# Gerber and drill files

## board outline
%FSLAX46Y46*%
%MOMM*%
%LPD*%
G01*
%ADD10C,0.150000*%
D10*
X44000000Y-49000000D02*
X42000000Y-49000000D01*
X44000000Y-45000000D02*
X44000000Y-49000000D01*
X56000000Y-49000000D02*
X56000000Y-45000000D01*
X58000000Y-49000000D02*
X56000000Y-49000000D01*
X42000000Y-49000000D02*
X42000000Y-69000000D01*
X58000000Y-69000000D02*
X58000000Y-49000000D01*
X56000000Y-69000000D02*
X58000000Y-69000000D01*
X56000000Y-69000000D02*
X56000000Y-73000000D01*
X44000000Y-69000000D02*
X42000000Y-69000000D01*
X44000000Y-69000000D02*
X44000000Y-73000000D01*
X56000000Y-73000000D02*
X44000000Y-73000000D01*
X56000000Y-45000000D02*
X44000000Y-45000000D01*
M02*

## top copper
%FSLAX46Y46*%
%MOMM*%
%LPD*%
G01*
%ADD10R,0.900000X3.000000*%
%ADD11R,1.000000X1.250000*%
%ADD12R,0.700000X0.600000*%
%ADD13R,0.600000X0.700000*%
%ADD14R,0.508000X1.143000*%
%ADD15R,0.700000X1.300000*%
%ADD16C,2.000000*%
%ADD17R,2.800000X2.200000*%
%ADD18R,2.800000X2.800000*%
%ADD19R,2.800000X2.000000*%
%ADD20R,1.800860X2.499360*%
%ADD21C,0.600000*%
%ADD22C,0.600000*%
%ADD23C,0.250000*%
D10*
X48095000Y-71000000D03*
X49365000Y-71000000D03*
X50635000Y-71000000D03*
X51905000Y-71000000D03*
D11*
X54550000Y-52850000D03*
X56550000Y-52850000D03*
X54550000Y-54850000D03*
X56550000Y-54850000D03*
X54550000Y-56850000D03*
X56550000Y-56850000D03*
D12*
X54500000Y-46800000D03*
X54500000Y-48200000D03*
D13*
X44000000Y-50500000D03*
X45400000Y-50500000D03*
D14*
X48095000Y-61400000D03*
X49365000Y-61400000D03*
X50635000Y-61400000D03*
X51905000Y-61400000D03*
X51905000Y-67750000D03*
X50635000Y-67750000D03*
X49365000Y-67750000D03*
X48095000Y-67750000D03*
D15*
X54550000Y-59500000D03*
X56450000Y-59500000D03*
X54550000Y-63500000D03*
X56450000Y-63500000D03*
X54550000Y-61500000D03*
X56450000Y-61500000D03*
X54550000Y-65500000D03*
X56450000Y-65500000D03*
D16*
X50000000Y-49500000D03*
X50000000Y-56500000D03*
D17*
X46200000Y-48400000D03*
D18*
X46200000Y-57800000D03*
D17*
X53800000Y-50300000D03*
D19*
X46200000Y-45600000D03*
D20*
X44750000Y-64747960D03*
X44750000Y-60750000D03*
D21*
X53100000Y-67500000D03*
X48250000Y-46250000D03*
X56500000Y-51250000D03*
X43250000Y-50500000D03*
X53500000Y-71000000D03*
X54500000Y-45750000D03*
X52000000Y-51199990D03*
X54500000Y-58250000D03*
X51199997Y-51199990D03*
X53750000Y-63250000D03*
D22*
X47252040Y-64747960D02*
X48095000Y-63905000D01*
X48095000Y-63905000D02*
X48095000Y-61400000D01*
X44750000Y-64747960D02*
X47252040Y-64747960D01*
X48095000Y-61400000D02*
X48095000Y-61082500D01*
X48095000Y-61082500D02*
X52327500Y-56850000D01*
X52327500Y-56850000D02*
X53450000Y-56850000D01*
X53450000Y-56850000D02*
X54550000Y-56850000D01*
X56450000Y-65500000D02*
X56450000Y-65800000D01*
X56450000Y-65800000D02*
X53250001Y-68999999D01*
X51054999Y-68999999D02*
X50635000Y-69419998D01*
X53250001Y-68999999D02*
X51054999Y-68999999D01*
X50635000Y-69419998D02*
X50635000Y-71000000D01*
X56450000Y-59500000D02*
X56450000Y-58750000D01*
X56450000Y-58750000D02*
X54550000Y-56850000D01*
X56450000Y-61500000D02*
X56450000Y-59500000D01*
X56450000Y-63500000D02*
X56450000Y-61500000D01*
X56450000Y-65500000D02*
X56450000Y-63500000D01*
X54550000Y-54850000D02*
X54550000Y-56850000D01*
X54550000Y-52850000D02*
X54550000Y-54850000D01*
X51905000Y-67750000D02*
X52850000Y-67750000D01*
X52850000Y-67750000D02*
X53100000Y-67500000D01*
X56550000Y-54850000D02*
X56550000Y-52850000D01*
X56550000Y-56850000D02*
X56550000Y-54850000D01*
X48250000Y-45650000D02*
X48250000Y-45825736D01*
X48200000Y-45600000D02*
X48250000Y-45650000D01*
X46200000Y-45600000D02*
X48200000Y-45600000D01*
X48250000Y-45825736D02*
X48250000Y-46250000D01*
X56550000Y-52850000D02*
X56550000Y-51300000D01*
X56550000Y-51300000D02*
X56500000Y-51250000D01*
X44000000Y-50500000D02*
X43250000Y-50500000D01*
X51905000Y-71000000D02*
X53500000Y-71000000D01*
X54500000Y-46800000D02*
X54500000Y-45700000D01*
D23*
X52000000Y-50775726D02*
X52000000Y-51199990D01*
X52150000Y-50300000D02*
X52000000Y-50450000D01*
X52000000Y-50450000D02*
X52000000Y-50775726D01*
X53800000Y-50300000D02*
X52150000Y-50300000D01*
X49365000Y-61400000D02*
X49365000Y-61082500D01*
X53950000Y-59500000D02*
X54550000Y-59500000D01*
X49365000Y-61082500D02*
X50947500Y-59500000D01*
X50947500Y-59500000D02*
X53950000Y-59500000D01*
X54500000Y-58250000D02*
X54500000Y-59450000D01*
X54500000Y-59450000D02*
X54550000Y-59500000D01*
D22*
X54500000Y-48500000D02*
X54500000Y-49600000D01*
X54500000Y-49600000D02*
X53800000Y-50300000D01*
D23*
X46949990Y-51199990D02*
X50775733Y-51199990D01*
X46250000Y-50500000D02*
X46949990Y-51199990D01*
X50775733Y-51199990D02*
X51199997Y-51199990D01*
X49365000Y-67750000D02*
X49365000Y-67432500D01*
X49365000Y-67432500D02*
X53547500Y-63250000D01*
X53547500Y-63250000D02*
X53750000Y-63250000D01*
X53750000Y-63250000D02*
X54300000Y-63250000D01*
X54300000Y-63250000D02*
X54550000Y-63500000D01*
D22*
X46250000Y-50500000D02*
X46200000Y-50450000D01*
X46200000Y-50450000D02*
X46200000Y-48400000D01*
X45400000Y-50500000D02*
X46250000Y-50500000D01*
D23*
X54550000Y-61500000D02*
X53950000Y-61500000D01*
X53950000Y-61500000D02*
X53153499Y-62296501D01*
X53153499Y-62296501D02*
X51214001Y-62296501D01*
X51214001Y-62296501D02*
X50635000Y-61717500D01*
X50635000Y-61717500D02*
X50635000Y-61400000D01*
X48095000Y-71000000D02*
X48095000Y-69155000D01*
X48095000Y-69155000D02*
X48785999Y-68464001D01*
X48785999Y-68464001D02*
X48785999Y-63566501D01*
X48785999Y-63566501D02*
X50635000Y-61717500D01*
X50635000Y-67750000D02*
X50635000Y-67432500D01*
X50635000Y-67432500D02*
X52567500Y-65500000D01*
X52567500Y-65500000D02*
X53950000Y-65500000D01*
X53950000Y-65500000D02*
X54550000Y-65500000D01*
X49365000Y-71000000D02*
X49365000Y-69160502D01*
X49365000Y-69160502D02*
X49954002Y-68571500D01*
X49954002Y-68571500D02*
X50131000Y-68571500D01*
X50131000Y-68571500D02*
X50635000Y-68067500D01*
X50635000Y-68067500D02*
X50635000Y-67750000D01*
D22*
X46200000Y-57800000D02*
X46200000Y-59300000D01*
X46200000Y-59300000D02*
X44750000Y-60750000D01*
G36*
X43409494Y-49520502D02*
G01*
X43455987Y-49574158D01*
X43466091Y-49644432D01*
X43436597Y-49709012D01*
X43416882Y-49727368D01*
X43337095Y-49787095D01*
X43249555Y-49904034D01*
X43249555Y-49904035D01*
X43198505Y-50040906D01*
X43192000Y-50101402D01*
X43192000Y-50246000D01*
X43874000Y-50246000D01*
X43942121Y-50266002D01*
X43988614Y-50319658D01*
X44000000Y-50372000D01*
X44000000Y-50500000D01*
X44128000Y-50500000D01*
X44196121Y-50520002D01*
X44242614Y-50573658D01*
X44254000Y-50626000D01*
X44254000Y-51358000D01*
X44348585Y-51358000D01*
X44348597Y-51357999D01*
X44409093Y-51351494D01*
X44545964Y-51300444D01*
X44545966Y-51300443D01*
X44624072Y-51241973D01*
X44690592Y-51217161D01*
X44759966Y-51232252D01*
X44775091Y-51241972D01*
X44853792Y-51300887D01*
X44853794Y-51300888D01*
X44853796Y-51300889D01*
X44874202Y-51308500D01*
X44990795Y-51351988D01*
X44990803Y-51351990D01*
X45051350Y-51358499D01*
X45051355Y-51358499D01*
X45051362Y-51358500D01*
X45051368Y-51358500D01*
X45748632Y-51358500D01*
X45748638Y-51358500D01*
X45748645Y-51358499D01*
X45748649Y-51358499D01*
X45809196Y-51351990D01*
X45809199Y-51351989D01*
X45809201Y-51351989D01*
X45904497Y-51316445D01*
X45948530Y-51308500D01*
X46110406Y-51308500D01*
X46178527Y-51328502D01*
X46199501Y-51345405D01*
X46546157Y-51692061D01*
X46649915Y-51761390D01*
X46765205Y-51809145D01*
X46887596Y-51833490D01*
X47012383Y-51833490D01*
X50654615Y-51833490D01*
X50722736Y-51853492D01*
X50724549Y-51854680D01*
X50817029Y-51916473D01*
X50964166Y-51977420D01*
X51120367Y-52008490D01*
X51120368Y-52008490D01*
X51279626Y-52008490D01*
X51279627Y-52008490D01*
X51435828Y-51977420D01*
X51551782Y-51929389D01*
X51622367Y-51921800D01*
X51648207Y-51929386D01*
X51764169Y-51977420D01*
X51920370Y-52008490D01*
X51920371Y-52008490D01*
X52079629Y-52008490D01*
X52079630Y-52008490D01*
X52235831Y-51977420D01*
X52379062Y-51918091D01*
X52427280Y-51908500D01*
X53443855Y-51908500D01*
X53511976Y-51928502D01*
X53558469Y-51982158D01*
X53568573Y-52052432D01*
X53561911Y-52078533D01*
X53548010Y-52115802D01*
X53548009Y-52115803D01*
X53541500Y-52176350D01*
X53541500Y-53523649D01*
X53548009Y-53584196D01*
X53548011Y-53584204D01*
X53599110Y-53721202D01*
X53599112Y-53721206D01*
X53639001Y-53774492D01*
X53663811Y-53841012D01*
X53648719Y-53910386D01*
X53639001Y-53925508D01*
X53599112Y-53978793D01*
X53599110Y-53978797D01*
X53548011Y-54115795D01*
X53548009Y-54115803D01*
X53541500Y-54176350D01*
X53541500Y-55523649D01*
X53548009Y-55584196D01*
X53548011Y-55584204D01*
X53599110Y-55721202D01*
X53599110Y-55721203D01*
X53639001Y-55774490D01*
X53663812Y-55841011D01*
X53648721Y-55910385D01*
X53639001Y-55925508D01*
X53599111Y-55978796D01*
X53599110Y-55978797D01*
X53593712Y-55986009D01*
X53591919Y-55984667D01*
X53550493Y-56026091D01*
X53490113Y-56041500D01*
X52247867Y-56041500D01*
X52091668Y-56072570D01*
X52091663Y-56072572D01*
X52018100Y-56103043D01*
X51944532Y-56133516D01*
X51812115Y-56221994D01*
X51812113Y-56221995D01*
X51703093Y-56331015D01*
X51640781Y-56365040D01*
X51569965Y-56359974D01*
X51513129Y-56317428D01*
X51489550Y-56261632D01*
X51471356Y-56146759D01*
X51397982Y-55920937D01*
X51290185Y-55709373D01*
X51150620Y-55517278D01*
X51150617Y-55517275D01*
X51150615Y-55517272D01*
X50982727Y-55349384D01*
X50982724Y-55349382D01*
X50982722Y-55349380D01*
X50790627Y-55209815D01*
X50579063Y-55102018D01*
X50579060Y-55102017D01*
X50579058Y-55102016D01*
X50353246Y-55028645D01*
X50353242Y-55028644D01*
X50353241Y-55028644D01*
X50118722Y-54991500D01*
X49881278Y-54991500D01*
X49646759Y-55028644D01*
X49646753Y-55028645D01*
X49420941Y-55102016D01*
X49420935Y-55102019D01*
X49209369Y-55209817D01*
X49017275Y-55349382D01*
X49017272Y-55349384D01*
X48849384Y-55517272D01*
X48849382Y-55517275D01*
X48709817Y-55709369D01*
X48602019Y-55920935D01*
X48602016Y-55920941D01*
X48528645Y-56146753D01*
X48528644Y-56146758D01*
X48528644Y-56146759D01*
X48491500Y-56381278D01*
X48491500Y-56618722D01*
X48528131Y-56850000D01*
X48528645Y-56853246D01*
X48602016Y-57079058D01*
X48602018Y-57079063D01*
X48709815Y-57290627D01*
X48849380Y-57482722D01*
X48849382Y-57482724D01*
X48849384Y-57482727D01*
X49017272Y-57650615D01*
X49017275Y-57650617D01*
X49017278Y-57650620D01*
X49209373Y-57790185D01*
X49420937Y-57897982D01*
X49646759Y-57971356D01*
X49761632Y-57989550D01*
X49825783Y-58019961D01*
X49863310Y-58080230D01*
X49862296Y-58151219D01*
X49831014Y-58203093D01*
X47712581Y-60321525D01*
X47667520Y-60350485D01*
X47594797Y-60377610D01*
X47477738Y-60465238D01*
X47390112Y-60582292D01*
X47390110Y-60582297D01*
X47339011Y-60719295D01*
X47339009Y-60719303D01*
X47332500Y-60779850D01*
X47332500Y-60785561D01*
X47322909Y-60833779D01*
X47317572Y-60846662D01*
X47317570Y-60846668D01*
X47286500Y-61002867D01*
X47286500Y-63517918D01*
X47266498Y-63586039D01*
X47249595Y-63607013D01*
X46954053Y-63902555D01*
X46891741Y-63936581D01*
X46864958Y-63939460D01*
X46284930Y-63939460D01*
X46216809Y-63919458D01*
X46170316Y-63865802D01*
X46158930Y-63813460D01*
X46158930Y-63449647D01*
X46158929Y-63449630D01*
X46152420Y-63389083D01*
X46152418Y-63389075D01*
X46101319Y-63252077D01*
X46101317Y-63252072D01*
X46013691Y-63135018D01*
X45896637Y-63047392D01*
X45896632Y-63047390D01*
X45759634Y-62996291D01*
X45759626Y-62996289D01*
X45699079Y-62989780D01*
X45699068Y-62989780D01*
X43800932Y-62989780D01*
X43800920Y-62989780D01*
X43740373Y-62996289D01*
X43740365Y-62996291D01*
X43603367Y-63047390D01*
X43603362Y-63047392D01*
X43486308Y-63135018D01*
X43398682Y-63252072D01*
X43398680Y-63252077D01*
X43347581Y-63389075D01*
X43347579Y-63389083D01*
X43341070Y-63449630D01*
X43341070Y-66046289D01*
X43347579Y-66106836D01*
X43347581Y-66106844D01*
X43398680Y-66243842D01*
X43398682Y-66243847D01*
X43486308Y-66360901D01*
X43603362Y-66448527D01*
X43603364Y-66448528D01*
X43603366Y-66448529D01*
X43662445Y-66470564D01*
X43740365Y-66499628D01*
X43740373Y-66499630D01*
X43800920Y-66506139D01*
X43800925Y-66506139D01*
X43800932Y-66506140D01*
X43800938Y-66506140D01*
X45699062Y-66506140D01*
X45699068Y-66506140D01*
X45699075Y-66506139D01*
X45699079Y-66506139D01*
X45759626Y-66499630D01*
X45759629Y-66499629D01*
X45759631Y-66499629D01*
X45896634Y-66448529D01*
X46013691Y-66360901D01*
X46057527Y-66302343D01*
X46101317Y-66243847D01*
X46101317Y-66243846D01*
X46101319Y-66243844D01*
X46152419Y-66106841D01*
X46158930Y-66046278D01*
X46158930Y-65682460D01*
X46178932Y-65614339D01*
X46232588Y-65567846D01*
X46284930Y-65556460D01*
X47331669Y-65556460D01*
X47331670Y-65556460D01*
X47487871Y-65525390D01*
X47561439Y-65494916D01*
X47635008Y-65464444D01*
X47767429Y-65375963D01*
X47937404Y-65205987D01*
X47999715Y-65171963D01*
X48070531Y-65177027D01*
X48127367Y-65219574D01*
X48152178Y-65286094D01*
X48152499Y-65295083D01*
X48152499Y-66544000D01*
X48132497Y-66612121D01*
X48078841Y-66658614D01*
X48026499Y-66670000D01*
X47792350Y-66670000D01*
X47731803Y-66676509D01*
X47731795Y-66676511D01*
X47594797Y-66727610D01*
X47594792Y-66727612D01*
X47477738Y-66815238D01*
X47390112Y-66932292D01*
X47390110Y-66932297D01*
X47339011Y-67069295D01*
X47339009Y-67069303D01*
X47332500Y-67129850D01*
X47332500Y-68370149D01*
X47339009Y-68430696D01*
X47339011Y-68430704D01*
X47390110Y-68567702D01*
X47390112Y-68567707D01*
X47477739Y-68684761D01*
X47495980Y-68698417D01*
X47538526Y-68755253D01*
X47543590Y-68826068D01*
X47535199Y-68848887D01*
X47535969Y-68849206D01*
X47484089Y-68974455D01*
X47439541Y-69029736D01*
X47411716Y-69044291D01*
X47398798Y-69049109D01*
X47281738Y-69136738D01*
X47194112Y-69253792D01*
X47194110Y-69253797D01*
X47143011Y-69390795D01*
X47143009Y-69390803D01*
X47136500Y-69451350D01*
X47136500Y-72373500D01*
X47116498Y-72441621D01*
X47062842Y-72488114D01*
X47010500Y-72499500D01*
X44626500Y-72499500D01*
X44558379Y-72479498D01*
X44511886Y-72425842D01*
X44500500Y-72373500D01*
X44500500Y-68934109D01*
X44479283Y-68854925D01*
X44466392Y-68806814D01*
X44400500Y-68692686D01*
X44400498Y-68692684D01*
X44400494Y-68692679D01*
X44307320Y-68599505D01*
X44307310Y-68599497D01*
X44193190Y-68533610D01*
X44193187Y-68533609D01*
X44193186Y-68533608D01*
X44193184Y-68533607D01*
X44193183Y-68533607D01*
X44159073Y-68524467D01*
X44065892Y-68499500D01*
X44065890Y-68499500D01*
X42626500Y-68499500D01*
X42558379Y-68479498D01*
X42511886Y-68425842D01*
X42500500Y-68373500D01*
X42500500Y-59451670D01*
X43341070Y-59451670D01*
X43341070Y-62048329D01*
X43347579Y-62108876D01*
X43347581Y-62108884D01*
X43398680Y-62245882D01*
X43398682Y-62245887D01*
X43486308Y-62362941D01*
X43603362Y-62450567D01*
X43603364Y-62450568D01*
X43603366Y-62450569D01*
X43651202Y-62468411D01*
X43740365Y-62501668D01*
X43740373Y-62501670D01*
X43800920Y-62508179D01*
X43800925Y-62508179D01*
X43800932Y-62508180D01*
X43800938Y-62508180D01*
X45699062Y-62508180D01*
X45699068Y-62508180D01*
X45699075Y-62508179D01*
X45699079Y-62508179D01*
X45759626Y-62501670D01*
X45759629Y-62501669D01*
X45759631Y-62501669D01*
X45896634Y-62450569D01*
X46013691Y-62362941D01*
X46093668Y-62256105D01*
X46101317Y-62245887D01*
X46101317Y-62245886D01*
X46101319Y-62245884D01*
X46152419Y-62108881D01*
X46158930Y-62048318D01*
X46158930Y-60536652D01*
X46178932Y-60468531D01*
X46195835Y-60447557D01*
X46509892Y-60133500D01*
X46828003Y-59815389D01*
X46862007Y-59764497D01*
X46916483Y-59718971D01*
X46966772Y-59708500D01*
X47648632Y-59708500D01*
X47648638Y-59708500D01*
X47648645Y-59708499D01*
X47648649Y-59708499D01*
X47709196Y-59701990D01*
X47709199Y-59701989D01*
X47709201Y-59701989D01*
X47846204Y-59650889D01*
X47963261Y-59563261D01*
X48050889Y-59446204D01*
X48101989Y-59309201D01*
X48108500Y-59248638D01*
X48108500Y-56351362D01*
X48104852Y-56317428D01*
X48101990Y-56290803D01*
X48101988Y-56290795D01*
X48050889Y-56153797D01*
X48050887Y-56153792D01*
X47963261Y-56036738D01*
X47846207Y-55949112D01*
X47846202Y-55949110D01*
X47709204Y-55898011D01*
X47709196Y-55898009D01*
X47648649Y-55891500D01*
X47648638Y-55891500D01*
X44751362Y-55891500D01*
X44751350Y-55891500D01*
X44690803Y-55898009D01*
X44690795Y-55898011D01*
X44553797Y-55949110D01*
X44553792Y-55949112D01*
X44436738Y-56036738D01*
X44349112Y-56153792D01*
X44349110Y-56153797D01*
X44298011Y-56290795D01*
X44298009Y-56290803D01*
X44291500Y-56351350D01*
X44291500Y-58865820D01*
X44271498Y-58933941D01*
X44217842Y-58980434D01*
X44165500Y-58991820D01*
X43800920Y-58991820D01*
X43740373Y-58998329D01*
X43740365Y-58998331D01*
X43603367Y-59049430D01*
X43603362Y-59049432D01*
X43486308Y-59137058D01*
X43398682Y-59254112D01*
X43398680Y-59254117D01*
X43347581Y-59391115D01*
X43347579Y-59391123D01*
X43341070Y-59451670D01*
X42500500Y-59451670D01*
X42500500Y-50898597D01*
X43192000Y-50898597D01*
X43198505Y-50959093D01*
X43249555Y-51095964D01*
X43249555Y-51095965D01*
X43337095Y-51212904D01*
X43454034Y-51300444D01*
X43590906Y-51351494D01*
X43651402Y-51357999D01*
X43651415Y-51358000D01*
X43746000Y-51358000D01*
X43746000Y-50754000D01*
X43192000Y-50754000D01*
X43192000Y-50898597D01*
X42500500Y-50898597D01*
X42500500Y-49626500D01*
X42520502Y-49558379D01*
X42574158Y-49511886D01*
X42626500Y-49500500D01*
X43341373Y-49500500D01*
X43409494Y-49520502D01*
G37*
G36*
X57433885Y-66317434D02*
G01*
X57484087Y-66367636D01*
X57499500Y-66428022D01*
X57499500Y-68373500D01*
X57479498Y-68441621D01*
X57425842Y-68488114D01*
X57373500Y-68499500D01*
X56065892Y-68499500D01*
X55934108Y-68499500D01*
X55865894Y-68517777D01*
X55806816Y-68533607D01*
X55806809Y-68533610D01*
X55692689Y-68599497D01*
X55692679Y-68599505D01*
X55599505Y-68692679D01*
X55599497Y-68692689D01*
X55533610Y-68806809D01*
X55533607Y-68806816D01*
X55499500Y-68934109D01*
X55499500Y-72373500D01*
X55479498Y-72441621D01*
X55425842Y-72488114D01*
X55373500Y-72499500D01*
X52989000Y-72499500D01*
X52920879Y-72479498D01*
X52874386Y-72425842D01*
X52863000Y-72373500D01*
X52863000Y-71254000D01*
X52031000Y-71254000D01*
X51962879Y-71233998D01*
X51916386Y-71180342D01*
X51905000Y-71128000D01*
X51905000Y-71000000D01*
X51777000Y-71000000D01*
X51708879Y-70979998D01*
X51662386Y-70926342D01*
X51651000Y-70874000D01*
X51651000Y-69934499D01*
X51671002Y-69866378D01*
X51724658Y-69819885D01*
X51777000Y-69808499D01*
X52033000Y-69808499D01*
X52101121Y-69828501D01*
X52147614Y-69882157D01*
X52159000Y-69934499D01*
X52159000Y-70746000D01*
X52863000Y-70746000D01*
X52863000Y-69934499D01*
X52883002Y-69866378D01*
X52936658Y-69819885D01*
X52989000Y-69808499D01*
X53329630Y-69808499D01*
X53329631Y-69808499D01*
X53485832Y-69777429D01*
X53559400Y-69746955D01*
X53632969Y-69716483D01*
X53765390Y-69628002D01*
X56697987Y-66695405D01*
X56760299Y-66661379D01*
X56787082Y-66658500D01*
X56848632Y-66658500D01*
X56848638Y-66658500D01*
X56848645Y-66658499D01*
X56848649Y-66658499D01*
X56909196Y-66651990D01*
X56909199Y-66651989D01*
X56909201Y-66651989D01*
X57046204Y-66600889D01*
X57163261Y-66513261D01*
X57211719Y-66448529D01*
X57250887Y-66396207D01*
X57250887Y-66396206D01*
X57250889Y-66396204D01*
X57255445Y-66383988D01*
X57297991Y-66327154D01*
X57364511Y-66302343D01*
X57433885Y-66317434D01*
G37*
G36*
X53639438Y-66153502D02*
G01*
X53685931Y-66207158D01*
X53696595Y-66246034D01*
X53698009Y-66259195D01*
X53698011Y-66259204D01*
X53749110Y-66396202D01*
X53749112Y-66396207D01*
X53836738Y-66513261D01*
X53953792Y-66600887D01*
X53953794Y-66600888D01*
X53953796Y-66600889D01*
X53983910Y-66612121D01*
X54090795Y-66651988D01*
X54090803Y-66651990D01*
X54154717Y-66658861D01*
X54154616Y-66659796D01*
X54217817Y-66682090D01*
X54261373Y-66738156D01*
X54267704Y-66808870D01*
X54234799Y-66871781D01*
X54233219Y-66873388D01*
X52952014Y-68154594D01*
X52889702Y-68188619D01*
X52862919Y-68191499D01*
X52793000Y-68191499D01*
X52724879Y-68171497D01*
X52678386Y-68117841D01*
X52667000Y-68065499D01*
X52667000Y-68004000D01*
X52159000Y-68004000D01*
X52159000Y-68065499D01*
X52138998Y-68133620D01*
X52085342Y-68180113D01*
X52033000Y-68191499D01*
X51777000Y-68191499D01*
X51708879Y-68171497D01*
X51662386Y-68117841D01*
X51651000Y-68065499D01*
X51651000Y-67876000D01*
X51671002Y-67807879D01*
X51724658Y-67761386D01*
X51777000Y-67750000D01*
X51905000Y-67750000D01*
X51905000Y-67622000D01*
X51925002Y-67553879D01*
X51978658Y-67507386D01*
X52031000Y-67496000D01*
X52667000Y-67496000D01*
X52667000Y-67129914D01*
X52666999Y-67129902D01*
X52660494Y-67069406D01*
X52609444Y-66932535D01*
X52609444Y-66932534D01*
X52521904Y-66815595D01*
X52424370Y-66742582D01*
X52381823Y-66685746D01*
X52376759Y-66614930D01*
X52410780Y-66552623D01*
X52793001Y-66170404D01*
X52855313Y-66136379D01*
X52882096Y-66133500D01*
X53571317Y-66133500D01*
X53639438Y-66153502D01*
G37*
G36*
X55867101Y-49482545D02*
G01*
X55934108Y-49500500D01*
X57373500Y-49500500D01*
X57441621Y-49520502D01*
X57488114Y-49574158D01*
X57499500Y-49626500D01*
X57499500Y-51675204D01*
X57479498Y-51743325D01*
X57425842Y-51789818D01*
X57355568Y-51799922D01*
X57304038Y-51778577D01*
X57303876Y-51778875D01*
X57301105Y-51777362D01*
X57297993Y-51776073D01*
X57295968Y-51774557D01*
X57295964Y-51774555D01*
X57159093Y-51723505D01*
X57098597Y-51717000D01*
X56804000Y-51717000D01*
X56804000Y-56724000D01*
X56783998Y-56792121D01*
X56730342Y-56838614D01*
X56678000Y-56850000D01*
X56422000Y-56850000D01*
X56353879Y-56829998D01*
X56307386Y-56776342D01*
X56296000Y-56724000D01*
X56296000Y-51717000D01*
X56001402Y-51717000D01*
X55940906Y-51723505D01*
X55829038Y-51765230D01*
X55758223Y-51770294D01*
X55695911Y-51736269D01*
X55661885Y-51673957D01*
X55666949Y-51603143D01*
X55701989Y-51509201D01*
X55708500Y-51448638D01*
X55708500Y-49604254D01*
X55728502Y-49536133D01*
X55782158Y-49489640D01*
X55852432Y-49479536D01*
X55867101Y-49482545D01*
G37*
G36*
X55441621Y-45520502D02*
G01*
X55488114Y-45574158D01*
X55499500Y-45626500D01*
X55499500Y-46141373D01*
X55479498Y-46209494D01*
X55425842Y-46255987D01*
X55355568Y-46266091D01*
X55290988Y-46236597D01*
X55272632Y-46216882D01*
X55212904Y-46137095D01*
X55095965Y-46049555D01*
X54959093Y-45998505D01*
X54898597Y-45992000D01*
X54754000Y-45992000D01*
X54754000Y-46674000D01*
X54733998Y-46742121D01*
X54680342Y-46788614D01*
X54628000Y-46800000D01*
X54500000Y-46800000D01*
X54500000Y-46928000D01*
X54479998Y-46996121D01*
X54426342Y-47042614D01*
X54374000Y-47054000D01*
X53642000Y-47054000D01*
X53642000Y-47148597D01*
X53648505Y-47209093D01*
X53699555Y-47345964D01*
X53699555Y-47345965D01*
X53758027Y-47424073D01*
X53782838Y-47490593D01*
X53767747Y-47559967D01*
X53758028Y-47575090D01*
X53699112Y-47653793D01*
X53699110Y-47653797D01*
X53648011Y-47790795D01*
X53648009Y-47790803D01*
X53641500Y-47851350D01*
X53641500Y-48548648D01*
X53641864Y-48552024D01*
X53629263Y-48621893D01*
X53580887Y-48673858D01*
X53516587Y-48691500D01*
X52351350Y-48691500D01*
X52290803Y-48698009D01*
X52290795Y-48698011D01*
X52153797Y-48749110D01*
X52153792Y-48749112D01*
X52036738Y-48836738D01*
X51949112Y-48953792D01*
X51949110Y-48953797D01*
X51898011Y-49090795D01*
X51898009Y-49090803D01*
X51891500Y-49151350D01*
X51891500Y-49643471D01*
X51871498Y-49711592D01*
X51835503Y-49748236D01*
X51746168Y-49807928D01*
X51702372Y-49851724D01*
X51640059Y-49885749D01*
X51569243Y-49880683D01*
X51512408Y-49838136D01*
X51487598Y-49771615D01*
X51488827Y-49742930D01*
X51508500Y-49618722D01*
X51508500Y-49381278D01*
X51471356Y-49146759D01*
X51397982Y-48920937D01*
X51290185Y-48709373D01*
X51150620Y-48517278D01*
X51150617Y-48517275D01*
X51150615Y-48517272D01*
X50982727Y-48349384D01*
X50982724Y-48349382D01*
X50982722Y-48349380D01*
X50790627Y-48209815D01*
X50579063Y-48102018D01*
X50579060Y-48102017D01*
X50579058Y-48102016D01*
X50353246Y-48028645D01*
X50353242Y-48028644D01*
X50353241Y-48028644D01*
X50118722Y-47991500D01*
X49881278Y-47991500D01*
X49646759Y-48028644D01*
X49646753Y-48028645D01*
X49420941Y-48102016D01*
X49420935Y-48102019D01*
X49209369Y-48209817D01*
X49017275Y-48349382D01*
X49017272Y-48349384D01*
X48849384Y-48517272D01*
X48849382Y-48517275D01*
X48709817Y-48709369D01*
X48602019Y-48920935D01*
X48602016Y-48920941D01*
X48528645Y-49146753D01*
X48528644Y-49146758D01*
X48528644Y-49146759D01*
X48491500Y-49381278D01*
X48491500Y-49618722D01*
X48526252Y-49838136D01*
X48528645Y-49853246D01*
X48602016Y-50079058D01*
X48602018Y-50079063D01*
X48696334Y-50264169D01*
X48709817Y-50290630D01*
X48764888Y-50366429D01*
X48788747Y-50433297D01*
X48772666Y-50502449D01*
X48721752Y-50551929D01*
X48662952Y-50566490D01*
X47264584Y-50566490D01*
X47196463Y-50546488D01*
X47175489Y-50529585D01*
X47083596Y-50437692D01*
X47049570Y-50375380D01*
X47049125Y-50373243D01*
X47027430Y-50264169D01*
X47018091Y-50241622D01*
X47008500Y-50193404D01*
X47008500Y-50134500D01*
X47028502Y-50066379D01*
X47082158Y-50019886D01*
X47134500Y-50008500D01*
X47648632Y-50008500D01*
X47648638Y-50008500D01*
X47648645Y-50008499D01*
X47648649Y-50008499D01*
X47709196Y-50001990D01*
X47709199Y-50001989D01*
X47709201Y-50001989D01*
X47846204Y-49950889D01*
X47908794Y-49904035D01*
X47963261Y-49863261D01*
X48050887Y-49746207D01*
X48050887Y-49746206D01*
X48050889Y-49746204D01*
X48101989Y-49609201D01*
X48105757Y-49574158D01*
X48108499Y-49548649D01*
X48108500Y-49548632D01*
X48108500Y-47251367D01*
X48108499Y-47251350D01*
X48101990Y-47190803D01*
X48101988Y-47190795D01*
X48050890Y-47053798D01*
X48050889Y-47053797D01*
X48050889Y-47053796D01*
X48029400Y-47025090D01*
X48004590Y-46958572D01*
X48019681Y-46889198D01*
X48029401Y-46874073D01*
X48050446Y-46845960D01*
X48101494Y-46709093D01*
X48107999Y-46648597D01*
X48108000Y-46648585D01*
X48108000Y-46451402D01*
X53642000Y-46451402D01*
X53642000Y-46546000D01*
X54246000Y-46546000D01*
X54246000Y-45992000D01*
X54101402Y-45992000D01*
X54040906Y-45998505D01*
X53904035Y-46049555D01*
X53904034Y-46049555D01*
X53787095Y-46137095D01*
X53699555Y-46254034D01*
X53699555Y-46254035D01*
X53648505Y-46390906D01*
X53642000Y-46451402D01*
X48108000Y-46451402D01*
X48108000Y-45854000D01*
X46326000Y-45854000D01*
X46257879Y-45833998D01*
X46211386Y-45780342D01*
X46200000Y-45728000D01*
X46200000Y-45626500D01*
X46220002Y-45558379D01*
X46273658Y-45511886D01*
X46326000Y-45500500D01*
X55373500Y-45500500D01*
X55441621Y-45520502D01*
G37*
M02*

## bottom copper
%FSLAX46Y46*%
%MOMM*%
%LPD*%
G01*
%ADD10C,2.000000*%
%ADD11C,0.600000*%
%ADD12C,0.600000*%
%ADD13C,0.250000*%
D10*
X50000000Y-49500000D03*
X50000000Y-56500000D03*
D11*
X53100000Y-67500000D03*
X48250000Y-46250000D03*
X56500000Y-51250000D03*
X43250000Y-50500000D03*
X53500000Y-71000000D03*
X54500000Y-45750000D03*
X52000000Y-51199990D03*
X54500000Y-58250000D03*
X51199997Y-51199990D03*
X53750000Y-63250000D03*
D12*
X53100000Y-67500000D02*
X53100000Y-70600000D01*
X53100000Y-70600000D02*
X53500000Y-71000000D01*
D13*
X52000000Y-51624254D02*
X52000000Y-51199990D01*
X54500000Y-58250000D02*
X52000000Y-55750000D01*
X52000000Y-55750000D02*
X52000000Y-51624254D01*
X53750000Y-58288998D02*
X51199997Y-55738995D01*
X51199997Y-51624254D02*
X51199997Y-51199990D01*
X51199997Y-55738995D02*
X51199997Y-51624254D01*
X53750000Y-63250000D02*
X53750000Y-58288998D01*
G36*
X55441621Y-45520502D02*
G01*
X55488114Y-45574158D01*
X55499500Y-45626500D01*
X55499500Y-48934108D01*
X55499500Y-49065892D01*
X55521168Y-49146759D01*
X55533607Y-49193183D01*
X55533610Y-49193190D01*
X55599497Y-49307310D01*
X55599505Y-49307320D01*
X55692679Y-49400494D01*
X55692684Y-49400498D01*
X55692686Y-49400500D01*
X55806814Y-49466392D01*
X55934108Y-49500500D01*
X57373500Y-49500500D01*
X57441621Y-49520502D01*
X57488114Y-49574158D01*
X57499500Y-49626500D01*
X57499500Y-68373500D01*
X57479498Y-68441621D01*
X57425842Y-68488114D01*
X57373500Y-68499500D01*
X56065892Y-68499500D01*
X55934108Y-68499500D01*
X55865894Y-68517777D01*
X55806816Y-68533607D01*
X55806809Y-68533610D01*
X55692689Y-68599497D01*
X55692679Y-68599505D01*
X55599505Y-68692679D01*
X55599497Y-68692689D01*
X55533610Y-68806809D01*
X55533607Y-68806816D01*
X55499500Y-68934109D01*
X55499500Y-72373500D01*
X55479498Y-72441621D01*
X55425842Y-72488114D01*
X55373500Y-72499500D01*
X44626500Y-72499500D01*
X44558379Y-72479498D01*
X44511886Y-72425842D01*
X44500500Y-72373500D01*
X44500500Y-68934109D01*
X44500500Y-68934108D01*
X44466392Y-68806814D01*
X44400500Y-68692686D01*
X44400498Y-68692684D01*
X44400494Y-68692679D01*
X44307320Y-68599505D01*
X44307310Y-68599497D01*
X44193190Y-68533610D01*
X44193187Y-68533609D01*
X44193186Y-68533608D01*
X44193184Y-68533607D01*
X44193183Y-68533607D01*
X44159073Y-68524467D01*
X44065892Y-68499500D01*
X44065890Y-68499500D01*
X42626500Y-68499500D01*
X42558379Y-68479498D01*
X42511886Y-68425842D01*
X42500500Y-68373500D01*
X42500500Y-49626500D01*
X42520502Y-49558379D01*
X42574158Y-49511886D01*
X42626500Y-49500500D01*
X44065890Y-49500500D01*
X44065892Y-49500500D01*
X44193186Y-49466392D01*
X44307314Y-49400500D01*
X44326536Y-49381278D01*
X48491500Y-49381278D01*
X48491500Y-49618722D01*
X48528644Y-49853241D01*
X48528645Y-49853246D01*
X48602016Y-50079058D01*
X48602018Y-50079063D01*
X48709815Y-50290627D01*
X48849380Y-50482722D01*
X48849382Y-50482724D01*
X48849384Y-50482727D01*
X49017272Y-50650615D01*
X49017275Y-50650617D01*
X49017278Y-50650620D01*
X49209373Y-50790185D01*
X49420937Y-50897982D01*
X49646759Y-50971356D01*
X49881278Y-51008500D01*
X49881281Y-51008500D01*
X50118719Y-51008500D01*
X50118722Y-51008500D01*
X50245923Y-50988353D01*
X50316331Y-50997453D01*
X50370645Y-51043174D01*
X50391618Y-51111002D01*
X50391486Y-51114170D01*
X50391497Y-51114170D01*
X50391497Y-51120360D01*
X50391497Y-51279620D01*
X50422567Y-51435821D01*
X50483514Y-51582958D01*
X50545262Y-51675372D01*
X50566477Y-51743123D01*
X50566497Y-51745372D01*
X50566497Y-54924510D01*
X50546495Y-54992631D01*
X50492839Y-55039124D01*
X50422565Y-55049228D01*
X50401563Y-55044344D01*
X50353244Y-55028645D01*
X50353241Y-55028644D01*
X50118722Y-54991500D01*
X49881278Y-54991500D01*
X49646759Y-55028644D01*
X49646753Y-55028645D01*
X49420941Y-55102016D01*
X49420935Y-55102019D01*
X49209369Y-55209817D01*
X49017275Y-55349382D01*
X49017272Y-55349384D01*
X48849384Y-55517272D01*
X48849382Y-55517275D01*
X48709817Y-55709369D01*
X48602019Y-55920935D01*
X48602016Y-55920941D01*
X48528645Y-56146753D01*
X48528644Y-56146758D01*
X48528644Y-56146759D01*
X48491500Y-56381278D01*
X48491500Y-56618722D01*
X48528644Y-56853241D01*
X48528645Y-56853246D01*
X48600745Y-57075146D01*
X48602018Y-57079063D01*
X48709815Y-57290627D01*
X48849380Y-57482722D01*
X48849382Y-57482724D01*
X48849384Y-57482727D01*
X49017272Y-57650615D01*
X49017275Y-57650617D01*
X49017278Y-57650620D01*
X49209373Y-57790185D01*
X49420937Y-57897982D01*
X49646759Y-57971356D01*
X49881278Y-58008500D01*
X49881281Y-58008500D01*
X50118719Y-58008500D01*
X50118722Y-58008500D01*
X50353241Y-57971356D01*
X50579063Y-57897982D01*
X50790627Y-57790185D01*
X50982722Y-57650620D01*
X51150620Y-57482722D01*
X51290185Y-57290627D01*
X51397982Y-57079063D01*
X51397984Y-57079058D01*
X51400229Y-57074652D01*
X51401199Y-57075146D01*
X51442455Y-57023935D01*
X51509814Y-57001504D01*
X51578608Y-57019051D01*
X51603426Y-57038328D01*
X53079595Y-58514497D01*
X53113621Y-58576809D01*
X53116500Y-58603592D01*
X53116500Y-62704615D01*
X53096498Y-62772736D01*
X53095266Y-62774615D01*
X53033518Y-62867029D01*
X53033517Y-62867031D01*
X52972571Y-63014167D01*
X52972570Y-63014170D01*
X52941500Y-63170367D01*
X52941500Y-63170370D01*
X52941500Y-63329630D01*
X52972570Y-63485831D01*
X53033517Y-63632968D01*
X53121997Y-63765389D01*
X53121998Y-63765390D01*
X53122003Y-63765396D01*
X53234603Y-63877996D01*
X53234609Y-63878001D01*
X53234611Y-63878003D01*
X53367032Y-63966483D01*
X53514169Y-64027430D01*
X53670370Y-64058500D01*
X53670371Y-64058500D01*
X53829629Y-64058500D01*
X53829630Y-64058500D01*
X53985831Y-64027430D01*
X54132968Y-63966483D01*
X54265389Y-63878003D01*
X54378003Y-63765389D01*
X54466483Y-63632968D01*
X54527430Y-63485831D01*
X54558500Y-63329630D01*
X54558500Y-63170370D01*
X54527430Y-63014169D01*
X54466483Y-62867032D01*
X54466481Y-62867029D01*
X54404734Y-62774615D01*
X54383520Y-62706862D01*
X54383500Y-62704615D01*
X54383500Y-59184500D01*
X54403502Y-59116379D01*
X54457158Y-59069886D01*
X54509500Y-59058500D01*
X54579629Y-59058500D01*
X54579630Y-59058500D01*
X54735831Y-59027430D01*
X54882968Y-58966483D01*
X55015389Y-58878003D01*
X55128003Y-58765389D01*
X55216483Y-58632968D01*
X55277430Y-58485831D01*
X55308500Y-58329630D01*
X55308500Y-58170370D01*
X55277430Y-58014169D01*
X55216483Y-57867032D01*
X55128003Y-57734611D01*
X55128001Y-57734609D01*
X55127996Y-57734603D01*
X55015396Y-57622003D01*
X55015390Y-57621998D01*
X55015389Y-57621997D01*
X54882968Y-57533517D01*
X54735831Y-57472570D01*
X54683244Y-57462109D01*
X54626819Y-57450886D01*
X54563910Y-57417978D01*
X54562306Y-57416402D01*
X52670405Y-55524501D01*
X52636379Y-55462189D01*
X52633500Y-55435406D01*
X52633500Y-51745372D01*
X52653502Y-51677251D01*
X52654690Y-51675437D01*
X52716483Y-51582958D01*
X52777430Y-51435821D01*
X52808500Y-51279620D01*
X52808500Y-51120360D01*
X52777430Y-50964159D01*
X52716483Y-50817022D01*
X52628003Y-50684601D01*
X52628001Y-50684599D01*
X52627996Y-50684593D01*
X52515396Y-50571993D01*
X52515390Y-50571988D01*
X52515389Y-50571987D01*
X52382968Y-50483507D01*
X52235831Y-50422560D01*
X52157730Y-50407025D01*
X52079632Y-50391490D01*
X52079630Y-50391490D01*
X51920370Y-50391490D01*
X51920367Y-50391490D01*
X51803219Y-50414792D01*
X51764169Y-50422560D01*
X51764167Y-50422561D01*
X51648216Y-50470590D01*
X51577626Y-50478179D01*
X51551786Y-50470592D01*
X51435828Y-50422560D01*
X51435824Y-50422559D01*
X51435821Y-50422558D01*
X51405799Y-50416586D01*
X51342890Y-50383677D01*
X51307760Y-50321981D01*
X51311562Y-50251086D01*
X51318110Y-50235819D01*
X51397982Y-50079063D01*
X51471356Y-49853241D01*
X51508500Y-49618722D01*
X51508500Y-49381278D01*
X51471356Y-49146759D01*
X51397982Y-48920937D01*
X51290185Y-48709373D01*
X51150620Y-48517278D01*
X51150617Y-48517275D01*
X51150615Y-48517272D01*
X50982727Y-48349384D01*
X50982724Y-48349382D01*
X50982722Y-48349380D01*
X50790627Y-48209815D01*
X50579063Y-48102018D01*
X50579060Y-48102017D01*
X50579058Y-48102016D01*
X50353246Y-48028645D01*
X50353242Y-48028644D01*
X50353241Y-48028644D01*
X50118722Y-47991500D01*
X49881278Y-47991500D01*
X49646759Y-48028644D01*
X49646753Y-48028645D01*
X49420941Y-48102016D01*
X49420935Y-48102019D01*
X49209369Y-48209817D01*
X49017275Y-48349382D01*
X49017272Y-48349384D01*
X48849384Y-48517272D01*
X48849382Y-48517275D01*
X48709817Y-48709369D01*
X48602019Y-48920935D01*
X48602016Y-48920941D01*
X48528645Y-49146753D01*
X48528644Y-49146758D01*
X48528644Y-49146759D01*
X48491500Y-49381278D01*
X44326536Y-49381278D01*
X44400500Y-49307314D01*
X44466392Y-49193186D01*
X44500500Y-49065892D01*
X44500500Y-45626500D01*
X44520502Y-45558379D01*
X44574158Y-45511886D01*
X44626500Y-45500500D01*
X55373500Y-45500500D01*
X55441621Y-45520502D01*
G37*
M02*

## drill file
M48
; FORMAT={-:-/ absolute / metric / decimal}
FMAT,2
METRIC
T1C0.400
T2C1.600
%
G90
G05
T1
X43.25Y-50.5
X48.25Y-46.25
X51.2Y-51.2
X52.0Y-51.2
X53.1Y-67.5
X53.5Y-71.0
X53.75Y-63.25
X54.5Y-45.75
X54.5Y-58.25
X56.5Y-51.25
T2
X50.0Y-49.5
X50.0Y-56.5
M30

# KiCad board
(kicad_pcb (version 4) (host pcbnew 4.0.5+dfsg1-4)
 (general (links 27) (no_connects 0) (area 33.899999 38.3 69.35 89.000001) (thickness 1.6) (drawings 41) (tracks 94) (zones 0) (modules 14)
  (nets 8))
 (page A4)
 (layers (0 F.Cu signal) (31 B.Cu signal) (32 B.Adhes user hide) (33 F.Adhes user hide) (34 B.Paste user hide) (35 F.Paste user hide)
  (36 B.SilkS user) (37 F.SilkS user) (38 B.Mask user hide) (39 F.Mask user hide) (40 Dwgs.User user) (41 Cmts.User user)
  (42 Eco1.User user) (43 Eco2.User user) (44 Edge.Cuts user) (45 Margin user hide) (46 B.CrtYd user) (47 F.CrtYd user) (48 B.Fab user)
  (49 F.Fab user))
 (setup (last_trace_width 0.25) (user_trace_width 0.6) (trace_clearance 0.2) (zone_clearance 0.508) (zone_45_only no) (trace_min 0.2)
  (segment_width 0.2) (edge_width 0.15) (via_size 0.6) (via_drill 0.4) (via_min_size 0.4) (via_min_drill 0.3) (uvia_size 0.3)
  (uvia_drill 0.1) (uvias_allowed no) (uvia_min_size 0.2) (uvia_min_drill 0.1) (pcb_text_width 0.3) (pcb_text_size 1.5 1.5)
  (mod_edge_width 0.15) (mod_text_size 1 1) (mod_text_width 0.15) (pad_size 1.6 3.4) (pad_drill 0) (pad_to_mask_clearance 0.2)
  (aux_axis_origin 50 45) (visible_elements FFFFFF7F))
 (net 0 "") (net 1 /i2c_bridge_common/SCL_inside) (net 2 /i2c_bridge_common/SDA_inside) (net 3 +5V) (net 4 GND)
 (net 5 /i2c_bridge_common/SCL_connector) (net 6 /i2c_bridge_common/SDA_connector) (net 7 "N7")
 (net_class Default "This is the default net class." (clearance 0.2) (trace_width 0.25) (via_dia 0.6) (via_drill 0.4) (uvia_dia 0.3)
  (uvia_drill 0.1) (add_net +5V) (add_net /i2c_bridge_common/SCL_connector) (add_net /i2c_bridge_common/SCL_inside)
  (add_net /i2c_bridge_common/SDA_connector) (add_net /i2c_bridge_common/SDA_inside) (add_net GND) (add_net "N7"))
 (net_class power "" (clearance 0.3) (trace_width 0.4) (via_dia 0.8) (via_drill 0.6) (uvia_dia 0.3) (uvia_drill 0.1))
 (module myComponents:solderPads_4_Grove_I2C (layer F.Cu) (at 50 71)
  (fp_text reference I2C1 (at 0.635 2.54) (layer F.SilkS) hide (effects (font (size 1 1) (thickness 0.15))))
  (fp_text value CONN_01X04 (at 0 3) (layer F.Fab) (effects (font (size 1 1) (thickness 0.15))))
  (pad 1 smd rect (at -1.905 0) (size 0.9 3) (layers F.Cu F.Paste F.Mask) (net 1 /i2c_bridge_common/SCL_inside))
  (pad 2 smd rect (at -0.635 0) (size 0.9 3) (layers F.Cu F.Paste F.Mask) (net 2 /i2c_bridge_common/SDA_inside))
  (pad 3 smd rect (at 0.635 0) (size 0.9 3) (layers F.Cu F.Paste F.Mask) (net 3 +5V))
  (pad 4 smd rect (at 1.905 0) (size 0.9 3) (layers F.Cu F.Paste F.Mask) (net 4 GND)))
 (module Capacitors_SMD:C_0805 (layer F.Cu) (at 55.55 52.85)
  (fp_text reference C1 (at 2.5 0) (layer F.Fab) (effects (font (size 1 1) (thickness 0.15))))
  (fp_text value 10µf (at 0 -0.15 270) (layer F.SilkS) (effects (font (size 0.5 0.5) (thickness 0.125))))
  (pad 1 smd rect (at -1 0) (size 1 1.25) (layers F.Cu F.Paste F.Mask) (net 3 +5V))
  (pad 2 smd rect (at 1 0) (size 1 1.25) (layers F.Cu F.Paste F.Mask) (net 4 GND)))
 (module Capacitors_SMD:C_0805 (layer F.Cu) (at 55.55 54.85)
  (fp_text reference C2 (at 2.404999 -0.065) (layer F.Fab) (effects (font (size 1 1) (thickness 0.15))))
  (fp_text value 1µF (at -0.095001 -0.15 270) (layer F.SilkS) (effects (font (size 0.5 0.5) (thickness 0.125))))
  (pad 1 smd rect (at -1 0) (size 1 1.25) (layers F.Cu F.Paste F.Mask) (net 3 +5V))
  (pad 2 smd rect (at 1 0) (size 1 1.25) (layers F.Cu F.Paste F.Mask) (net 4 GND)))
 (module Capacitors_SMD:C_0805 (layer F.Cu) (at 55.55 56.85)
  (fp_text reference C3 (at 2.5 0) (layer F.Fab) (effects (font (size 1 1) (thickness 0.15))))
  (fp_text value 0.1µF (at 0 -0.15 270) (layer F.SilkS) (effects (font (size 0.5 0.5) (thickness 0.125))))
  (pad 1 smd rect (at -1 0) (size 1 1.25) (layers F.Cu F.Paste F.Mask) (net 3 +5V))
  (pad 2 smd rect (at 1 0) (size 1 1.25) (layers F.Cu F.Paste F.Mask) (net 4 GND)))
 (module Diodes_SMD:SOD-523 (layer F.Cu) (at 54.5 47.5 90)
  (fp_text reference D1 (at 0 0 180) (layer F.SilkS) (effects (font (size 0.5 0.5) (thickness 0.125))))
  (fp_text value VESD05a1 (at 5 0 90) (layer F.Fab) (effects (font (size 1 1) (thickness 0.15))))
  (pad 2 smd rect (at 0.7 0 270) (size 0.6 0.7) (layers F.Cu F.Paste F.Mask) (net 4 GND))
  (pad 1 smd rect (at -0.7 0 270) (size 0.6 0.7) (layers F.Cu F.Paste F.Mask) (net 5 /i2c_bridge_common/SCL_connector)))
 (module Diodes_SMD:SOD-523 (layer F.Cu) (at 44.7 50.5 180)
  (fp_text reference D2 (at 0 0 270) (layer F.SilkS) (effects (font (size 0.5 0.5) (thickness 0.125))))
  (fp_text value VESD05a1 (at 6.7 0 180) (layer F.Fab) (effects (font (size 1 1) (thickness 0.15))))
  (pad 2 smd rect (at 0.7 0) (size 0.6 0.7) (layers F.Cu F.Paste F.Mask) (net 4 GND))
  (pad 1 smd rect (at -0.7 0) (size 0.6 0.7) (layers F.Cu F.Paste F.Mask) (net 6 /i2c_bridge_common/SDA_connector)))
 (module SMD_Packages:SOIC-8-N (layer F.Cu) (at 50 64.575)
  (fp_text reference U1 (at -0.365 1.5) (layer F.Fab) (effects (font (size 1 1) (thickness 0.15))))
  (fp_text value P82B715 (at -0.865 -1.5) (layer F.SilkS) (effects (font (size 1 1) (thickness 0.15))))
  (pad 8 smd rect (at -1.905 -3.175) (size 0.508 1.143) (layers F.Cu F.Paste F.Mask) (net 3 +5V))
  (pad 7 smd rect (at -0.635 -3.175) (size 0.508 1.143) (layers F.Cu F.Paste F.Mask) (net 5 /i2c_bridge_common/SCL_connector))
  (pad 6 smd rect (at 0.635 -3.175) (size 0.508 1.143) (layers F.Cu F.Paste F.Mask) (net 1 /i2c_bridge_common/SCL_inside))
  (pad 5 smd rect (at 1.905 -3.175) (size 0.508 1.143) (layers F.Cu F.Paste F.Mask))
  (pad 4 smd rect (at 1.905 3.175) (size 0.508 1.143) (layers F.Cu F.Paste F.Mask) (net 4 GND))
  (pad 3 smd rect (at 0.635 3.175) (size 0.508 1.143) (layers F.Cu F.Paste F.Mask) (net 2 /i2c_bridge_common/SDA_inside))
  (pad 2 smd rect (at -0.635 3.175) (size 0.508 1.143) (layers F.Cu F.Paste F.Mask) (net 6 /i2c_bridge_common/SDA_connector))
  (pad 1 smd rect (at -1.905 3.175) (size 0.508 1.143) (layers F.Cu F.Paste F.Mask)))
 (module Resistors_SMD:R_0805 (layer F.Cu) (at 55.5 59.5)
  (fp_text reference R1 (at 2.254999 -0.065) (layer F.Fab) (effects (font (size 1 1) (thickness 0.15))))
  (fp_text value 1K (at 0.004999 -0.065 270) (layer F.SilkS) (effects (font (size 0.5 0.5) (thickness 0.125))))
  (pad 1 smd rect (at -0.95 0) (size 0.7 1.3) (layers F.Cu F.Paste F.Mask) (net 5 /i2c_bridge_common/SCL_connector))
  (pad 2 smd rect (at 0.95 0) (size 0.7 1.3) (layers F.Cu F.Paste F.Mask) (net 3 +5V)))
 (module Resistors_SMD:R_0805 (layer F.Cu) (at 55.5 63.5)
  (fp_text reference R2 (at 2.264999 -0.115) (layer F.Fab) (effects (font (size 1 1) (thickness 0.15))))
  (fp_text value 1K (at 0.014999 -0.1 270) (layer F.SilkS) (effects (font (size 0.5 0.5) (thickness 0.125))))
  (pad 1 smd rect (at -0.95 0) (size 0.7 1.3) (layers F.Cu F.Paste F.Mask) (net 6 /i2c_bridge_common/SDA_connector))
  (pad 2 smd rect (at 0.95 0) (size 0.7 1.3) (layers F.Cu F.Paste F.Mask) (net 3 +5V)))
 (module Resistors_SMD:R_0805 (layer F.Cu) (at 55.5 61.5)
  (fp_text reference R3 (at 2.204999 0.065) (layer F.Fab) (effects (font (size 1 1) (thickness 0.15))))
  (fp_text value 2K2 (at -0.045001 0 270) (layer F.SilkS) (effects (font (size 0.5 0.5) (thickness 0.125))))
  (pad 1 smd rect (at -0.95 0) (size 0.7 1.3) (layers F.Cu F.Paste F.Mask) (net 1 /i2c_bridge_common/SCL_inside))
  (pad 2 smd rect (at 0.95 0) (size 0.7 1.3) (layers F.Cu F.Paste F.Mask) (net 3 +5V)))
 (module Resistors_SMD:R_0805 (layer F.Cu) (at 55.5 65.5)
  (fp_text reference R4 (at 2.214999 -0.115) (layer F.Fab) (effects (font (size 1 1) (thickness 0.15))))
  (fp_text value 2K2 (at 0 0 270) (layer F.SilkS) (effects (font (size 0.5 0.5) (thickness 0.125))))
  (pad 1 smd rect (at -0.95 0) (size 0.7 1.3) (layers F.Cu F.Paste F.Mask) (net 2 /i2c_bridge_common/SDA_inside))
  (pad 2 smd rect (at 0.95 0) (size 0.7 1.3) (layers F.Cu F.Paste F.Mask) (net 3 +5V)))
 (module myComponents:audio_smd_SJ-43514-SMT (layer F.Cu) (at 50 45 270)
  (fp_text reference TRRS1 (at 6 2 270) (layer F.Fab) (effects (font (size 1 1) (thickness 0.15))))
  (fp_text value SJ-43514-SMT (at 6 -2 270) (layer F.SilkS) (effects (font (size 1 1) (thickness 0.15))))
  (pad "" thru_hole circle (at 4.5 0 270) (size 2 2) (drill 1.6) (layers *.Cu *.Mask F.SilkS))
  (pad "" thru_hole circle (at 11.5 0 270) (size 2 2) (drill 1.6) (layers *.Cu *.Mask F.SilkS))
  (pad 4 smd rect (at 3.4 3.8 270) (size 2.2 2.8) (layers F.Cu F.Paste F.Mask) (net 6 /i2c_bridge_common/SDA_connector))
  (pad 2 smd rect (at 12.8 3.8 270) (size 2.8 2.8) (layers F.Cu F.Paste F.Mask) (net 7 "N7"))
  (pad 3 smd rect (at 5.3 -3.8 270) (size 2.2 2.8) (layers F.Cu F.Paste F.Mask) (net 5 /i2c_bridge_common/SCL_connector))
  (pad 1 smd rect (at 0.6 3.8 270) (size 2 2.8) (layers F.Cu F.Paste F.Mask) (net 4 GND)))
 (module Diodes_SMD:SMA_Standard (layer F.Cu) (at 44.75 62.74898 90)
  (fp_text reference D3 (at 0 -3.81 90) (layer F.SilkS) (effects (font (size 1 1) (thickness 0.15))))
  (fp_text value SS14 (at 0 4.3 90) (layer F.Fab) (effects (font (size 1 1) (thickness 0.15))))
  (pad 1 smd rect (at -1.99898 0 90) (size 2.49936 1.80086) (layers F.Cu F.Paste F.Mask) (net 3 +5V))
  (pad 2 smd rect (at 1.99898 0 90) (size 2.49936 1.80086) (layers F.Cu F.Paste F.Mask) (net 7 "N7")))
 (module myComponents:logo (layer B.Cu) (at 50 64.2 180)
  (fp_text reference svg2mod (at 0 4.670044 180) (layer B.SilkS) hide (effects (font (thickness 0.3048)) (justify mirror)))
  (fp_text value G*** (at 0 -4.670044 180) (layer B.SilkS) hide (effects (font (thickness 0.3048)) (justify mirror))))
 (gr_line (start 44 49) (end 42 49) (layer Edge.Cuts) (width 0.15))
 (gr_line (start 44 45) (end 44 49) (layer Edge.Cuts) (width 0.15))
 (gr_line (start 56 49) (end 56 45) (layer Edge.Cuts) (width 0.15))
 (gr_line (start 58 49) (end 56 49) (layer Edge.Cuts) (width 0.15))
 (gr_line (start 42 49) (end 42 69) (layer Edge.Cuts) (width 0.15))
 (gr_line (start 58 69) (end 58 49) (layer Edge.Cuts) (width 0.15))
 (gr_line (start 56 69) (end 58 69) (layer Edge.Cuts) (width 0.15))
 (gr_line (start 56 69) (end 56 73) (layer Edge.Cuts) (width 0.15))
 (gr_line (start 44 69) (end 42 69) (layer Edge.Cuts) (width 0.15))
 (gr_line (start 44 69) (end 44 73) (layer Edge.Cuts) (width 0.15))
 (gr_line (start 56 73) (end 44 73) (layer Edge.Cuts) (width 0.15))
 (gr_line (start 56 45) (end 44 45) (layer Edge.Cuts) (width 0.15))
 (segment (start 47.25204 64.74796) (end 48.095 63.905) (width 0.6) (layer F.Cu) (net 3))
 (segment (start 48.095 63.905) (end 48.095 61.4) (width 0.6) (layer F.Cu) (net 3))
 (segment (start 44.75 64.74796) (end 47.25204 64.74796) (width 0.6) (layer F.Cu) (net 3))
 (segment (start 48.095 61.4) (end 48.095 61.0825) (width 0.6) (layer F.Cu) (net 3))
 (segment (start 48.095 61.0825) (end 52.3275 56.85) (width 0.6) (layer F.Cu) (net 3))
 (segment (start 52.3275 56.85) (end 53.45 56.85) (width 0.6) (layer F.Cu) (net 3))
 (segment (start 53.45 56.85) (end 54.55 56.85) (width 0.6) (layer F.Cu) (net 3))
 (segment (start 56.45 65.5) (end 56.45 65.8) (width 0.6) (layer F.Cu) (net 3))
 (segment (start 56.45 65.8) (end 53.250001 68.999999) (width 0.6) (layer F.Cu) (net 3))
 (segment (start 51.054999 68.999999) (end 50.635 69.419998) (width 0.6) (layer F.Cu) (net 3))
 (segment (start 53.250001 68.999999) (end 51.054999 68.999999) (width 0.6) (layer F.Cu) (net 3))
 (segment (start 50.635 69.419998) (end 50.635 71) (width 0.6) (layer F.Cu) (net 3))
 (segment (start 56.45 59.5) (end 56.45 58.75) (width 0.6) (layer F.Cu) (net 3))
 (segment (start 56.45 58.75) (end 54.55 56.85) (width 0.6) (layer F.Cu) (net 3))
 (segment (start 56.45 61.5) (end 56.45 59.5) (width 0.6) (layer F.Cu) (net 3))
 (segment (start 56.45 63.5) (end 56.45 61.5) (width 0.6) (layer F.Cu) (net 3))
 (segment (start 56.45 65.5) (end 56.45 63.5) (width 0.6) (layer F.Cu) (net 3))
 (segment (start 54.55 54.85) (end 54.55 56.85) (width 0.6) (layer F.Cu) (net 3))
 (segment (start 54.55 52.85) (end 54.55 54.85) (width 0.6) (layer F.Cu) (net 3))
 (segment (start 53.1 67.5) (end 53.1 70.6) (width 0.6) (layer B.Cu) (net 4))
 (segment (start 53.1 70.6) (end 53.5 71) (width 0.6) (layer B.Cu) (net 4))
 (segment (start 51.905 67.75) (end 52.85 67.75) (width 0.6) (layer F.Cu) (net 4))
 (segment (start 52.85 67.75) (end 53.1 67.5) (width 0.6) (layer F.Cu) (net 4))
 (via (at 53.1 67.5) (size 0.6) (drill 0.4) (layers F.Cu B.Cu) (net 4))
 (segment (start 56.55 54.85) (end 56.55 52.85) (width 0.6) (layer F.Cu) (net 4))
 (segment (start 56.55 56.85) (end 56.55 54.85) (width 0.6) (layer F.Cu) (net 4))
 (segment (start 48.25 45.65) (end 48.25 45.825736) (width 0.6) (layer F.Cu) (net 4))
 (segment (start 48.2 45.6) (end 48.25 45.65) (width 0.6) (layer F.Cu) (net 4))
 (segment (start 46.2 45.6) (end 48.2 45.6) (width 0.6) (layer F.Cu) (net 4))
 (segment (start 48.25 45.825736) (end 48.25 46.25) (width 0.6) (layer F.Cu) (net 4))
 (via (at 48.25 46.25) (size 0.6) (drill 0.4) (layers F.Cu B.Cu) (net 4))
 (segment (start 56.55 52.85) (end 56.55 51.3) (width 0.6) (layer F.Cu) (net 4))
 (segment (start 56.55 51.3) (end 56.5 51.25) (width 0.6) (layer F.Cu) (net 4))
 (via (at 56.5 51.25) (size 0.6) (drill 0.4) (layers F.Cu B.Cu) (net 4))
 (segment (start 44 50.5) (end 43.25 50.5) (width 0.6) (layer F.Cu) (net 4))
 (via (at 43.25 50.5) (size 0.6) (drill 0.4) (layers F.Cu B.Cu) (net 4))
 (segment (start 51.905 71) (end 53.5 71) (width 0.6) (layer F.Cu) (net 4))
 (via (at 53.5 71) (size 0.6) (drill 0.4) (layers F.Cu B.Cu) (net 4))
 (segment (start 54.5 46.8) (end 54.5 45.7) (width 0.6) (layer F.Cu) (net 4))
 (via (at 54.5 45.75) (size 0.6) (drill 0.4) (layers F.Cu B.Cu) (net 4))
 (segment (start 52 50.775726) (end 52 51.19999) (width 0.25) (layer F.Cu) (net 5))
 (segment (start 52.15 50.3) (end 52 50.45) (width 0.25) (layer F.Cu) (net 5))
 (segment (start 52 50.45) (end 52 50.775726) (width 0.25) (layer F.Cu) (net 5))
 (via (at 52 51.19999) (size 0.6) (drill 0.4) (layers F.Cu B.Cu) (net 5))
 (segment (start 52 51.624254) (end 52 51.19999) (width 0.25) (layer B.Cu) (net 5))
 (segment (start 54.5 58.25) (end 52 55.75) (width 0.25) (layer B.Cu) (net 5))
 (segment (start 52 55.75) (end 52 51.624254) (width 0.25) (layer B.Cu) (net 5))
 (segment (start 53.8 50.3) (end 52.15 50.3) (width 0.25) (layer F.Cu) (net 5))
 (segment (start 49.365 61.4) (end 49.365 61.0825) (width 0.25) (layer F.Cu) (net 5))
 (segment (start 53.95 59.5) (end 54.55 59.5) (width 0.25) (layer F.Cu) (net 5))
 (segment (start 49.365 61.0825) (end 50.9475 59.5) (width 0.25) (layer F.Cu) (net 5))
 (segment (start 50.9475 59.5) (end 53.95 59.5) (width 0.25) (layer F.Cu) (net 5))
 (segment (start 54.5 58.25) (end 54.5 59.45) (width 0.25) (layer F.Cu) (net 5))
 (segment (start 54.5 59.45) (end 54.55 59.5) (width 0.25) (layer F.Cu) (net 5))
 (via (at 54.5 58.25) (size 0.6) (drill 0.4) (layers F.Cu B.Cu) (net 5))
 (segment (start 54.5 48.5) (end 54.5 49.6) (width 0.6) (layer F.Cu) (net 5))
 (segment (start 54.5 49.6) (end 53.8 50.3) (width 0.6) (layer F.Cu) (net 5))
 (segment (start 53.75 58.288998) (end 51.199997 55.738995) (width 0.25) (layer B.Cu) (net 6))
 (segment (start 46.94999 51.19999) (end 50.775733 51.19999) (width 0.25) (layer F.Cu) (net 6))
 (segment (start 46.25 50.5) (end 46.94999 51.19999) (width 0.25) (layer F.Cu) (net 6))
 (segment (start 51.199997 51.624254) (end 51.199997 51.19999) (width 0.25) (layer B.Cu) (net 6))
 (segment (start 51.199997 55.738995) (end 51.199997 51.624254) (width 0.25) (layer B.Cu) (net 6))
 (segment (start 50.775733 51.19999) (end 51.199997 51.19999) (width 0.25) (layer F.Cu) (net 6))
 (segment (start 53.75 63.25) (end 53.75 58.288998) (width 0.25) (layer B.Cu) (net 6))
 (via (at 51.199997 51.19999) (size 0.6) (drill 0.4) (layers F.Cu B.Cu) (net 6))
 (segment (start 49.365 67.75) (end 49.365 67.4325) (width 0.25) (layer F.Cu) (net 6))
 (segment (start 49.365 67.4325) (end 53.5475 63.25) (width 0.25) (layer F.Cu) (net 6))
 (segment (start 53.5475 63.25) (end 53.75 63.25) (width 0.25) (layer F.Cu) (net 6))
 (segment (start 53.75 63.25) (end 54.3 63.25) (width 0.25) (layer F.Cu) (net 6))
 (segment (start 54.3 63.25) (end 54.55 63.5) (width 0.25) (layer F.Cu) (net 6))
 (via (at 53.75 63.25) (size 0.6) (drill 0.4) (layers F.Cu B.Cu) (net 6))
 (segment (start 46.25 50.5) (end 46.2 50.45) (width 0.6) (layer F.Cu) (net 6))
 (segment (start 46.2 50.45) (end 46.2 48.4) (width 0.6) (layer F.Cu) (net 6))
 (segment (start 45.4 50.5) (end 46.25 50.5) (width 0.6) (layer F.Cu) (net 6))
 (segment (start 54.55 61.5) (end 53.95 61.5) (width 0.25) (layer F.Cu) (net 1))
 (segment (start 53.95 61.5) (end 53.153499 62.296501) (width 0.25) (layer F.Cu) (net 1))
 (segment (start 53.153499 62.296501) (end 51.214001 62.296501) (width 0.25) (layer F.Cu) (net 1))
 (segment (start 51.214001 62.296501) (end 50.635 61.7175) (width 0.25) (layer F.Cu) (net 1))
 (segment (start 50.635 61.7175) (end 50.635 61.4) (width 0.25) (layer F.Cu) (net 1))
 (segment (start 48.095 71) (end 48.095 69.155) (width 0.25) (layer F.Cu) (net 1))
 (segment (start 48.095 69.155) (end 48.785999 68.464001) (width 0.25) (layer F.Cu) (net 1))
 (segment (start 48.785999 68.464001) (end 48.785999 63.566501) (width 0.25) (layer F.Cu) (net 1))
 (segment (start 48.785999 63.566501) (end 50.635 61.7175) (width 0.25) (layer F.Cu) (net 1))
 (segment (start 50.635 67.75) (end 50.635 67.4325) (width 0.25) (layer F.Cu) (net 2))
 (segment (start 50.635 67.4325) (end 52.5675 65.5) (width 0.25) (layer F.Cu) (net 2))
 (segment (start 52.5675 65.5) (end 53.95 65.5) (width 0.25) (layer F.Cu) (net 2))
 (segment (start 53.95 65.5) (end 54.55 65.5) (width 0.25) (layer F.Cu) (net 2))
 (segment (start 49.365 71) (end 49.365 69.160502) (width 0.25) (layer F.Cu) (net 2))
 (segment (start 49.365 69.160502) (end 49.954002 68.5715) (width 0.25) (layer F.Cu) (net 2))
 (segment (start 49.954002 68.5715) (end 50.131 68.5715) (width 0.25) (layer F.Cu) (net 2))
 (segment (start 50.131 68.5715) (end 50.635 68.0675) (width 0.25) (layer F.Cu) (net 2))
 (segment (start 50.635 68.0675) (end 50.635 67.75) (width 0.25) (layer F.Cu) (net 2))
 (segment (start 46.2 57.8) (end 46.2 59.3) (width 0.6) (layer F.Cu) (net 7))
 (segment (start 46.2 59.3) (end 44.75 60.75) (width 0.6) (layer F.Cu) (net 7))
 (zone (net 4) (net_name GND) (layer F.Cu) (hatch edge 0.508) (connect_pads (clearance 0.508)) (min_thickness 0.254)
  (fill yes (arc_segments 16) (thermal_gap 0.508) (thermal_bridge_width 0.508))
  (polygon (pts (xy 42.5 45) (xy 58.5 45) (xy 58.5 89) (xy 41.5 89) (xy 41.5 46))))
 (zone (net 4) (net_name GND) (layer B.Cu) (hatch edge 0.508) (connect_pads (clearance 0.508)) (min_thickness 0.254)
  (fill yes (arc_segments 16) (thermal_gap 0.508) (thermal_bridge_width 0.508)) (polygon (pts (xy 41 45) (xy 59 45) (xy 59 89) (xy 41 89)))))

